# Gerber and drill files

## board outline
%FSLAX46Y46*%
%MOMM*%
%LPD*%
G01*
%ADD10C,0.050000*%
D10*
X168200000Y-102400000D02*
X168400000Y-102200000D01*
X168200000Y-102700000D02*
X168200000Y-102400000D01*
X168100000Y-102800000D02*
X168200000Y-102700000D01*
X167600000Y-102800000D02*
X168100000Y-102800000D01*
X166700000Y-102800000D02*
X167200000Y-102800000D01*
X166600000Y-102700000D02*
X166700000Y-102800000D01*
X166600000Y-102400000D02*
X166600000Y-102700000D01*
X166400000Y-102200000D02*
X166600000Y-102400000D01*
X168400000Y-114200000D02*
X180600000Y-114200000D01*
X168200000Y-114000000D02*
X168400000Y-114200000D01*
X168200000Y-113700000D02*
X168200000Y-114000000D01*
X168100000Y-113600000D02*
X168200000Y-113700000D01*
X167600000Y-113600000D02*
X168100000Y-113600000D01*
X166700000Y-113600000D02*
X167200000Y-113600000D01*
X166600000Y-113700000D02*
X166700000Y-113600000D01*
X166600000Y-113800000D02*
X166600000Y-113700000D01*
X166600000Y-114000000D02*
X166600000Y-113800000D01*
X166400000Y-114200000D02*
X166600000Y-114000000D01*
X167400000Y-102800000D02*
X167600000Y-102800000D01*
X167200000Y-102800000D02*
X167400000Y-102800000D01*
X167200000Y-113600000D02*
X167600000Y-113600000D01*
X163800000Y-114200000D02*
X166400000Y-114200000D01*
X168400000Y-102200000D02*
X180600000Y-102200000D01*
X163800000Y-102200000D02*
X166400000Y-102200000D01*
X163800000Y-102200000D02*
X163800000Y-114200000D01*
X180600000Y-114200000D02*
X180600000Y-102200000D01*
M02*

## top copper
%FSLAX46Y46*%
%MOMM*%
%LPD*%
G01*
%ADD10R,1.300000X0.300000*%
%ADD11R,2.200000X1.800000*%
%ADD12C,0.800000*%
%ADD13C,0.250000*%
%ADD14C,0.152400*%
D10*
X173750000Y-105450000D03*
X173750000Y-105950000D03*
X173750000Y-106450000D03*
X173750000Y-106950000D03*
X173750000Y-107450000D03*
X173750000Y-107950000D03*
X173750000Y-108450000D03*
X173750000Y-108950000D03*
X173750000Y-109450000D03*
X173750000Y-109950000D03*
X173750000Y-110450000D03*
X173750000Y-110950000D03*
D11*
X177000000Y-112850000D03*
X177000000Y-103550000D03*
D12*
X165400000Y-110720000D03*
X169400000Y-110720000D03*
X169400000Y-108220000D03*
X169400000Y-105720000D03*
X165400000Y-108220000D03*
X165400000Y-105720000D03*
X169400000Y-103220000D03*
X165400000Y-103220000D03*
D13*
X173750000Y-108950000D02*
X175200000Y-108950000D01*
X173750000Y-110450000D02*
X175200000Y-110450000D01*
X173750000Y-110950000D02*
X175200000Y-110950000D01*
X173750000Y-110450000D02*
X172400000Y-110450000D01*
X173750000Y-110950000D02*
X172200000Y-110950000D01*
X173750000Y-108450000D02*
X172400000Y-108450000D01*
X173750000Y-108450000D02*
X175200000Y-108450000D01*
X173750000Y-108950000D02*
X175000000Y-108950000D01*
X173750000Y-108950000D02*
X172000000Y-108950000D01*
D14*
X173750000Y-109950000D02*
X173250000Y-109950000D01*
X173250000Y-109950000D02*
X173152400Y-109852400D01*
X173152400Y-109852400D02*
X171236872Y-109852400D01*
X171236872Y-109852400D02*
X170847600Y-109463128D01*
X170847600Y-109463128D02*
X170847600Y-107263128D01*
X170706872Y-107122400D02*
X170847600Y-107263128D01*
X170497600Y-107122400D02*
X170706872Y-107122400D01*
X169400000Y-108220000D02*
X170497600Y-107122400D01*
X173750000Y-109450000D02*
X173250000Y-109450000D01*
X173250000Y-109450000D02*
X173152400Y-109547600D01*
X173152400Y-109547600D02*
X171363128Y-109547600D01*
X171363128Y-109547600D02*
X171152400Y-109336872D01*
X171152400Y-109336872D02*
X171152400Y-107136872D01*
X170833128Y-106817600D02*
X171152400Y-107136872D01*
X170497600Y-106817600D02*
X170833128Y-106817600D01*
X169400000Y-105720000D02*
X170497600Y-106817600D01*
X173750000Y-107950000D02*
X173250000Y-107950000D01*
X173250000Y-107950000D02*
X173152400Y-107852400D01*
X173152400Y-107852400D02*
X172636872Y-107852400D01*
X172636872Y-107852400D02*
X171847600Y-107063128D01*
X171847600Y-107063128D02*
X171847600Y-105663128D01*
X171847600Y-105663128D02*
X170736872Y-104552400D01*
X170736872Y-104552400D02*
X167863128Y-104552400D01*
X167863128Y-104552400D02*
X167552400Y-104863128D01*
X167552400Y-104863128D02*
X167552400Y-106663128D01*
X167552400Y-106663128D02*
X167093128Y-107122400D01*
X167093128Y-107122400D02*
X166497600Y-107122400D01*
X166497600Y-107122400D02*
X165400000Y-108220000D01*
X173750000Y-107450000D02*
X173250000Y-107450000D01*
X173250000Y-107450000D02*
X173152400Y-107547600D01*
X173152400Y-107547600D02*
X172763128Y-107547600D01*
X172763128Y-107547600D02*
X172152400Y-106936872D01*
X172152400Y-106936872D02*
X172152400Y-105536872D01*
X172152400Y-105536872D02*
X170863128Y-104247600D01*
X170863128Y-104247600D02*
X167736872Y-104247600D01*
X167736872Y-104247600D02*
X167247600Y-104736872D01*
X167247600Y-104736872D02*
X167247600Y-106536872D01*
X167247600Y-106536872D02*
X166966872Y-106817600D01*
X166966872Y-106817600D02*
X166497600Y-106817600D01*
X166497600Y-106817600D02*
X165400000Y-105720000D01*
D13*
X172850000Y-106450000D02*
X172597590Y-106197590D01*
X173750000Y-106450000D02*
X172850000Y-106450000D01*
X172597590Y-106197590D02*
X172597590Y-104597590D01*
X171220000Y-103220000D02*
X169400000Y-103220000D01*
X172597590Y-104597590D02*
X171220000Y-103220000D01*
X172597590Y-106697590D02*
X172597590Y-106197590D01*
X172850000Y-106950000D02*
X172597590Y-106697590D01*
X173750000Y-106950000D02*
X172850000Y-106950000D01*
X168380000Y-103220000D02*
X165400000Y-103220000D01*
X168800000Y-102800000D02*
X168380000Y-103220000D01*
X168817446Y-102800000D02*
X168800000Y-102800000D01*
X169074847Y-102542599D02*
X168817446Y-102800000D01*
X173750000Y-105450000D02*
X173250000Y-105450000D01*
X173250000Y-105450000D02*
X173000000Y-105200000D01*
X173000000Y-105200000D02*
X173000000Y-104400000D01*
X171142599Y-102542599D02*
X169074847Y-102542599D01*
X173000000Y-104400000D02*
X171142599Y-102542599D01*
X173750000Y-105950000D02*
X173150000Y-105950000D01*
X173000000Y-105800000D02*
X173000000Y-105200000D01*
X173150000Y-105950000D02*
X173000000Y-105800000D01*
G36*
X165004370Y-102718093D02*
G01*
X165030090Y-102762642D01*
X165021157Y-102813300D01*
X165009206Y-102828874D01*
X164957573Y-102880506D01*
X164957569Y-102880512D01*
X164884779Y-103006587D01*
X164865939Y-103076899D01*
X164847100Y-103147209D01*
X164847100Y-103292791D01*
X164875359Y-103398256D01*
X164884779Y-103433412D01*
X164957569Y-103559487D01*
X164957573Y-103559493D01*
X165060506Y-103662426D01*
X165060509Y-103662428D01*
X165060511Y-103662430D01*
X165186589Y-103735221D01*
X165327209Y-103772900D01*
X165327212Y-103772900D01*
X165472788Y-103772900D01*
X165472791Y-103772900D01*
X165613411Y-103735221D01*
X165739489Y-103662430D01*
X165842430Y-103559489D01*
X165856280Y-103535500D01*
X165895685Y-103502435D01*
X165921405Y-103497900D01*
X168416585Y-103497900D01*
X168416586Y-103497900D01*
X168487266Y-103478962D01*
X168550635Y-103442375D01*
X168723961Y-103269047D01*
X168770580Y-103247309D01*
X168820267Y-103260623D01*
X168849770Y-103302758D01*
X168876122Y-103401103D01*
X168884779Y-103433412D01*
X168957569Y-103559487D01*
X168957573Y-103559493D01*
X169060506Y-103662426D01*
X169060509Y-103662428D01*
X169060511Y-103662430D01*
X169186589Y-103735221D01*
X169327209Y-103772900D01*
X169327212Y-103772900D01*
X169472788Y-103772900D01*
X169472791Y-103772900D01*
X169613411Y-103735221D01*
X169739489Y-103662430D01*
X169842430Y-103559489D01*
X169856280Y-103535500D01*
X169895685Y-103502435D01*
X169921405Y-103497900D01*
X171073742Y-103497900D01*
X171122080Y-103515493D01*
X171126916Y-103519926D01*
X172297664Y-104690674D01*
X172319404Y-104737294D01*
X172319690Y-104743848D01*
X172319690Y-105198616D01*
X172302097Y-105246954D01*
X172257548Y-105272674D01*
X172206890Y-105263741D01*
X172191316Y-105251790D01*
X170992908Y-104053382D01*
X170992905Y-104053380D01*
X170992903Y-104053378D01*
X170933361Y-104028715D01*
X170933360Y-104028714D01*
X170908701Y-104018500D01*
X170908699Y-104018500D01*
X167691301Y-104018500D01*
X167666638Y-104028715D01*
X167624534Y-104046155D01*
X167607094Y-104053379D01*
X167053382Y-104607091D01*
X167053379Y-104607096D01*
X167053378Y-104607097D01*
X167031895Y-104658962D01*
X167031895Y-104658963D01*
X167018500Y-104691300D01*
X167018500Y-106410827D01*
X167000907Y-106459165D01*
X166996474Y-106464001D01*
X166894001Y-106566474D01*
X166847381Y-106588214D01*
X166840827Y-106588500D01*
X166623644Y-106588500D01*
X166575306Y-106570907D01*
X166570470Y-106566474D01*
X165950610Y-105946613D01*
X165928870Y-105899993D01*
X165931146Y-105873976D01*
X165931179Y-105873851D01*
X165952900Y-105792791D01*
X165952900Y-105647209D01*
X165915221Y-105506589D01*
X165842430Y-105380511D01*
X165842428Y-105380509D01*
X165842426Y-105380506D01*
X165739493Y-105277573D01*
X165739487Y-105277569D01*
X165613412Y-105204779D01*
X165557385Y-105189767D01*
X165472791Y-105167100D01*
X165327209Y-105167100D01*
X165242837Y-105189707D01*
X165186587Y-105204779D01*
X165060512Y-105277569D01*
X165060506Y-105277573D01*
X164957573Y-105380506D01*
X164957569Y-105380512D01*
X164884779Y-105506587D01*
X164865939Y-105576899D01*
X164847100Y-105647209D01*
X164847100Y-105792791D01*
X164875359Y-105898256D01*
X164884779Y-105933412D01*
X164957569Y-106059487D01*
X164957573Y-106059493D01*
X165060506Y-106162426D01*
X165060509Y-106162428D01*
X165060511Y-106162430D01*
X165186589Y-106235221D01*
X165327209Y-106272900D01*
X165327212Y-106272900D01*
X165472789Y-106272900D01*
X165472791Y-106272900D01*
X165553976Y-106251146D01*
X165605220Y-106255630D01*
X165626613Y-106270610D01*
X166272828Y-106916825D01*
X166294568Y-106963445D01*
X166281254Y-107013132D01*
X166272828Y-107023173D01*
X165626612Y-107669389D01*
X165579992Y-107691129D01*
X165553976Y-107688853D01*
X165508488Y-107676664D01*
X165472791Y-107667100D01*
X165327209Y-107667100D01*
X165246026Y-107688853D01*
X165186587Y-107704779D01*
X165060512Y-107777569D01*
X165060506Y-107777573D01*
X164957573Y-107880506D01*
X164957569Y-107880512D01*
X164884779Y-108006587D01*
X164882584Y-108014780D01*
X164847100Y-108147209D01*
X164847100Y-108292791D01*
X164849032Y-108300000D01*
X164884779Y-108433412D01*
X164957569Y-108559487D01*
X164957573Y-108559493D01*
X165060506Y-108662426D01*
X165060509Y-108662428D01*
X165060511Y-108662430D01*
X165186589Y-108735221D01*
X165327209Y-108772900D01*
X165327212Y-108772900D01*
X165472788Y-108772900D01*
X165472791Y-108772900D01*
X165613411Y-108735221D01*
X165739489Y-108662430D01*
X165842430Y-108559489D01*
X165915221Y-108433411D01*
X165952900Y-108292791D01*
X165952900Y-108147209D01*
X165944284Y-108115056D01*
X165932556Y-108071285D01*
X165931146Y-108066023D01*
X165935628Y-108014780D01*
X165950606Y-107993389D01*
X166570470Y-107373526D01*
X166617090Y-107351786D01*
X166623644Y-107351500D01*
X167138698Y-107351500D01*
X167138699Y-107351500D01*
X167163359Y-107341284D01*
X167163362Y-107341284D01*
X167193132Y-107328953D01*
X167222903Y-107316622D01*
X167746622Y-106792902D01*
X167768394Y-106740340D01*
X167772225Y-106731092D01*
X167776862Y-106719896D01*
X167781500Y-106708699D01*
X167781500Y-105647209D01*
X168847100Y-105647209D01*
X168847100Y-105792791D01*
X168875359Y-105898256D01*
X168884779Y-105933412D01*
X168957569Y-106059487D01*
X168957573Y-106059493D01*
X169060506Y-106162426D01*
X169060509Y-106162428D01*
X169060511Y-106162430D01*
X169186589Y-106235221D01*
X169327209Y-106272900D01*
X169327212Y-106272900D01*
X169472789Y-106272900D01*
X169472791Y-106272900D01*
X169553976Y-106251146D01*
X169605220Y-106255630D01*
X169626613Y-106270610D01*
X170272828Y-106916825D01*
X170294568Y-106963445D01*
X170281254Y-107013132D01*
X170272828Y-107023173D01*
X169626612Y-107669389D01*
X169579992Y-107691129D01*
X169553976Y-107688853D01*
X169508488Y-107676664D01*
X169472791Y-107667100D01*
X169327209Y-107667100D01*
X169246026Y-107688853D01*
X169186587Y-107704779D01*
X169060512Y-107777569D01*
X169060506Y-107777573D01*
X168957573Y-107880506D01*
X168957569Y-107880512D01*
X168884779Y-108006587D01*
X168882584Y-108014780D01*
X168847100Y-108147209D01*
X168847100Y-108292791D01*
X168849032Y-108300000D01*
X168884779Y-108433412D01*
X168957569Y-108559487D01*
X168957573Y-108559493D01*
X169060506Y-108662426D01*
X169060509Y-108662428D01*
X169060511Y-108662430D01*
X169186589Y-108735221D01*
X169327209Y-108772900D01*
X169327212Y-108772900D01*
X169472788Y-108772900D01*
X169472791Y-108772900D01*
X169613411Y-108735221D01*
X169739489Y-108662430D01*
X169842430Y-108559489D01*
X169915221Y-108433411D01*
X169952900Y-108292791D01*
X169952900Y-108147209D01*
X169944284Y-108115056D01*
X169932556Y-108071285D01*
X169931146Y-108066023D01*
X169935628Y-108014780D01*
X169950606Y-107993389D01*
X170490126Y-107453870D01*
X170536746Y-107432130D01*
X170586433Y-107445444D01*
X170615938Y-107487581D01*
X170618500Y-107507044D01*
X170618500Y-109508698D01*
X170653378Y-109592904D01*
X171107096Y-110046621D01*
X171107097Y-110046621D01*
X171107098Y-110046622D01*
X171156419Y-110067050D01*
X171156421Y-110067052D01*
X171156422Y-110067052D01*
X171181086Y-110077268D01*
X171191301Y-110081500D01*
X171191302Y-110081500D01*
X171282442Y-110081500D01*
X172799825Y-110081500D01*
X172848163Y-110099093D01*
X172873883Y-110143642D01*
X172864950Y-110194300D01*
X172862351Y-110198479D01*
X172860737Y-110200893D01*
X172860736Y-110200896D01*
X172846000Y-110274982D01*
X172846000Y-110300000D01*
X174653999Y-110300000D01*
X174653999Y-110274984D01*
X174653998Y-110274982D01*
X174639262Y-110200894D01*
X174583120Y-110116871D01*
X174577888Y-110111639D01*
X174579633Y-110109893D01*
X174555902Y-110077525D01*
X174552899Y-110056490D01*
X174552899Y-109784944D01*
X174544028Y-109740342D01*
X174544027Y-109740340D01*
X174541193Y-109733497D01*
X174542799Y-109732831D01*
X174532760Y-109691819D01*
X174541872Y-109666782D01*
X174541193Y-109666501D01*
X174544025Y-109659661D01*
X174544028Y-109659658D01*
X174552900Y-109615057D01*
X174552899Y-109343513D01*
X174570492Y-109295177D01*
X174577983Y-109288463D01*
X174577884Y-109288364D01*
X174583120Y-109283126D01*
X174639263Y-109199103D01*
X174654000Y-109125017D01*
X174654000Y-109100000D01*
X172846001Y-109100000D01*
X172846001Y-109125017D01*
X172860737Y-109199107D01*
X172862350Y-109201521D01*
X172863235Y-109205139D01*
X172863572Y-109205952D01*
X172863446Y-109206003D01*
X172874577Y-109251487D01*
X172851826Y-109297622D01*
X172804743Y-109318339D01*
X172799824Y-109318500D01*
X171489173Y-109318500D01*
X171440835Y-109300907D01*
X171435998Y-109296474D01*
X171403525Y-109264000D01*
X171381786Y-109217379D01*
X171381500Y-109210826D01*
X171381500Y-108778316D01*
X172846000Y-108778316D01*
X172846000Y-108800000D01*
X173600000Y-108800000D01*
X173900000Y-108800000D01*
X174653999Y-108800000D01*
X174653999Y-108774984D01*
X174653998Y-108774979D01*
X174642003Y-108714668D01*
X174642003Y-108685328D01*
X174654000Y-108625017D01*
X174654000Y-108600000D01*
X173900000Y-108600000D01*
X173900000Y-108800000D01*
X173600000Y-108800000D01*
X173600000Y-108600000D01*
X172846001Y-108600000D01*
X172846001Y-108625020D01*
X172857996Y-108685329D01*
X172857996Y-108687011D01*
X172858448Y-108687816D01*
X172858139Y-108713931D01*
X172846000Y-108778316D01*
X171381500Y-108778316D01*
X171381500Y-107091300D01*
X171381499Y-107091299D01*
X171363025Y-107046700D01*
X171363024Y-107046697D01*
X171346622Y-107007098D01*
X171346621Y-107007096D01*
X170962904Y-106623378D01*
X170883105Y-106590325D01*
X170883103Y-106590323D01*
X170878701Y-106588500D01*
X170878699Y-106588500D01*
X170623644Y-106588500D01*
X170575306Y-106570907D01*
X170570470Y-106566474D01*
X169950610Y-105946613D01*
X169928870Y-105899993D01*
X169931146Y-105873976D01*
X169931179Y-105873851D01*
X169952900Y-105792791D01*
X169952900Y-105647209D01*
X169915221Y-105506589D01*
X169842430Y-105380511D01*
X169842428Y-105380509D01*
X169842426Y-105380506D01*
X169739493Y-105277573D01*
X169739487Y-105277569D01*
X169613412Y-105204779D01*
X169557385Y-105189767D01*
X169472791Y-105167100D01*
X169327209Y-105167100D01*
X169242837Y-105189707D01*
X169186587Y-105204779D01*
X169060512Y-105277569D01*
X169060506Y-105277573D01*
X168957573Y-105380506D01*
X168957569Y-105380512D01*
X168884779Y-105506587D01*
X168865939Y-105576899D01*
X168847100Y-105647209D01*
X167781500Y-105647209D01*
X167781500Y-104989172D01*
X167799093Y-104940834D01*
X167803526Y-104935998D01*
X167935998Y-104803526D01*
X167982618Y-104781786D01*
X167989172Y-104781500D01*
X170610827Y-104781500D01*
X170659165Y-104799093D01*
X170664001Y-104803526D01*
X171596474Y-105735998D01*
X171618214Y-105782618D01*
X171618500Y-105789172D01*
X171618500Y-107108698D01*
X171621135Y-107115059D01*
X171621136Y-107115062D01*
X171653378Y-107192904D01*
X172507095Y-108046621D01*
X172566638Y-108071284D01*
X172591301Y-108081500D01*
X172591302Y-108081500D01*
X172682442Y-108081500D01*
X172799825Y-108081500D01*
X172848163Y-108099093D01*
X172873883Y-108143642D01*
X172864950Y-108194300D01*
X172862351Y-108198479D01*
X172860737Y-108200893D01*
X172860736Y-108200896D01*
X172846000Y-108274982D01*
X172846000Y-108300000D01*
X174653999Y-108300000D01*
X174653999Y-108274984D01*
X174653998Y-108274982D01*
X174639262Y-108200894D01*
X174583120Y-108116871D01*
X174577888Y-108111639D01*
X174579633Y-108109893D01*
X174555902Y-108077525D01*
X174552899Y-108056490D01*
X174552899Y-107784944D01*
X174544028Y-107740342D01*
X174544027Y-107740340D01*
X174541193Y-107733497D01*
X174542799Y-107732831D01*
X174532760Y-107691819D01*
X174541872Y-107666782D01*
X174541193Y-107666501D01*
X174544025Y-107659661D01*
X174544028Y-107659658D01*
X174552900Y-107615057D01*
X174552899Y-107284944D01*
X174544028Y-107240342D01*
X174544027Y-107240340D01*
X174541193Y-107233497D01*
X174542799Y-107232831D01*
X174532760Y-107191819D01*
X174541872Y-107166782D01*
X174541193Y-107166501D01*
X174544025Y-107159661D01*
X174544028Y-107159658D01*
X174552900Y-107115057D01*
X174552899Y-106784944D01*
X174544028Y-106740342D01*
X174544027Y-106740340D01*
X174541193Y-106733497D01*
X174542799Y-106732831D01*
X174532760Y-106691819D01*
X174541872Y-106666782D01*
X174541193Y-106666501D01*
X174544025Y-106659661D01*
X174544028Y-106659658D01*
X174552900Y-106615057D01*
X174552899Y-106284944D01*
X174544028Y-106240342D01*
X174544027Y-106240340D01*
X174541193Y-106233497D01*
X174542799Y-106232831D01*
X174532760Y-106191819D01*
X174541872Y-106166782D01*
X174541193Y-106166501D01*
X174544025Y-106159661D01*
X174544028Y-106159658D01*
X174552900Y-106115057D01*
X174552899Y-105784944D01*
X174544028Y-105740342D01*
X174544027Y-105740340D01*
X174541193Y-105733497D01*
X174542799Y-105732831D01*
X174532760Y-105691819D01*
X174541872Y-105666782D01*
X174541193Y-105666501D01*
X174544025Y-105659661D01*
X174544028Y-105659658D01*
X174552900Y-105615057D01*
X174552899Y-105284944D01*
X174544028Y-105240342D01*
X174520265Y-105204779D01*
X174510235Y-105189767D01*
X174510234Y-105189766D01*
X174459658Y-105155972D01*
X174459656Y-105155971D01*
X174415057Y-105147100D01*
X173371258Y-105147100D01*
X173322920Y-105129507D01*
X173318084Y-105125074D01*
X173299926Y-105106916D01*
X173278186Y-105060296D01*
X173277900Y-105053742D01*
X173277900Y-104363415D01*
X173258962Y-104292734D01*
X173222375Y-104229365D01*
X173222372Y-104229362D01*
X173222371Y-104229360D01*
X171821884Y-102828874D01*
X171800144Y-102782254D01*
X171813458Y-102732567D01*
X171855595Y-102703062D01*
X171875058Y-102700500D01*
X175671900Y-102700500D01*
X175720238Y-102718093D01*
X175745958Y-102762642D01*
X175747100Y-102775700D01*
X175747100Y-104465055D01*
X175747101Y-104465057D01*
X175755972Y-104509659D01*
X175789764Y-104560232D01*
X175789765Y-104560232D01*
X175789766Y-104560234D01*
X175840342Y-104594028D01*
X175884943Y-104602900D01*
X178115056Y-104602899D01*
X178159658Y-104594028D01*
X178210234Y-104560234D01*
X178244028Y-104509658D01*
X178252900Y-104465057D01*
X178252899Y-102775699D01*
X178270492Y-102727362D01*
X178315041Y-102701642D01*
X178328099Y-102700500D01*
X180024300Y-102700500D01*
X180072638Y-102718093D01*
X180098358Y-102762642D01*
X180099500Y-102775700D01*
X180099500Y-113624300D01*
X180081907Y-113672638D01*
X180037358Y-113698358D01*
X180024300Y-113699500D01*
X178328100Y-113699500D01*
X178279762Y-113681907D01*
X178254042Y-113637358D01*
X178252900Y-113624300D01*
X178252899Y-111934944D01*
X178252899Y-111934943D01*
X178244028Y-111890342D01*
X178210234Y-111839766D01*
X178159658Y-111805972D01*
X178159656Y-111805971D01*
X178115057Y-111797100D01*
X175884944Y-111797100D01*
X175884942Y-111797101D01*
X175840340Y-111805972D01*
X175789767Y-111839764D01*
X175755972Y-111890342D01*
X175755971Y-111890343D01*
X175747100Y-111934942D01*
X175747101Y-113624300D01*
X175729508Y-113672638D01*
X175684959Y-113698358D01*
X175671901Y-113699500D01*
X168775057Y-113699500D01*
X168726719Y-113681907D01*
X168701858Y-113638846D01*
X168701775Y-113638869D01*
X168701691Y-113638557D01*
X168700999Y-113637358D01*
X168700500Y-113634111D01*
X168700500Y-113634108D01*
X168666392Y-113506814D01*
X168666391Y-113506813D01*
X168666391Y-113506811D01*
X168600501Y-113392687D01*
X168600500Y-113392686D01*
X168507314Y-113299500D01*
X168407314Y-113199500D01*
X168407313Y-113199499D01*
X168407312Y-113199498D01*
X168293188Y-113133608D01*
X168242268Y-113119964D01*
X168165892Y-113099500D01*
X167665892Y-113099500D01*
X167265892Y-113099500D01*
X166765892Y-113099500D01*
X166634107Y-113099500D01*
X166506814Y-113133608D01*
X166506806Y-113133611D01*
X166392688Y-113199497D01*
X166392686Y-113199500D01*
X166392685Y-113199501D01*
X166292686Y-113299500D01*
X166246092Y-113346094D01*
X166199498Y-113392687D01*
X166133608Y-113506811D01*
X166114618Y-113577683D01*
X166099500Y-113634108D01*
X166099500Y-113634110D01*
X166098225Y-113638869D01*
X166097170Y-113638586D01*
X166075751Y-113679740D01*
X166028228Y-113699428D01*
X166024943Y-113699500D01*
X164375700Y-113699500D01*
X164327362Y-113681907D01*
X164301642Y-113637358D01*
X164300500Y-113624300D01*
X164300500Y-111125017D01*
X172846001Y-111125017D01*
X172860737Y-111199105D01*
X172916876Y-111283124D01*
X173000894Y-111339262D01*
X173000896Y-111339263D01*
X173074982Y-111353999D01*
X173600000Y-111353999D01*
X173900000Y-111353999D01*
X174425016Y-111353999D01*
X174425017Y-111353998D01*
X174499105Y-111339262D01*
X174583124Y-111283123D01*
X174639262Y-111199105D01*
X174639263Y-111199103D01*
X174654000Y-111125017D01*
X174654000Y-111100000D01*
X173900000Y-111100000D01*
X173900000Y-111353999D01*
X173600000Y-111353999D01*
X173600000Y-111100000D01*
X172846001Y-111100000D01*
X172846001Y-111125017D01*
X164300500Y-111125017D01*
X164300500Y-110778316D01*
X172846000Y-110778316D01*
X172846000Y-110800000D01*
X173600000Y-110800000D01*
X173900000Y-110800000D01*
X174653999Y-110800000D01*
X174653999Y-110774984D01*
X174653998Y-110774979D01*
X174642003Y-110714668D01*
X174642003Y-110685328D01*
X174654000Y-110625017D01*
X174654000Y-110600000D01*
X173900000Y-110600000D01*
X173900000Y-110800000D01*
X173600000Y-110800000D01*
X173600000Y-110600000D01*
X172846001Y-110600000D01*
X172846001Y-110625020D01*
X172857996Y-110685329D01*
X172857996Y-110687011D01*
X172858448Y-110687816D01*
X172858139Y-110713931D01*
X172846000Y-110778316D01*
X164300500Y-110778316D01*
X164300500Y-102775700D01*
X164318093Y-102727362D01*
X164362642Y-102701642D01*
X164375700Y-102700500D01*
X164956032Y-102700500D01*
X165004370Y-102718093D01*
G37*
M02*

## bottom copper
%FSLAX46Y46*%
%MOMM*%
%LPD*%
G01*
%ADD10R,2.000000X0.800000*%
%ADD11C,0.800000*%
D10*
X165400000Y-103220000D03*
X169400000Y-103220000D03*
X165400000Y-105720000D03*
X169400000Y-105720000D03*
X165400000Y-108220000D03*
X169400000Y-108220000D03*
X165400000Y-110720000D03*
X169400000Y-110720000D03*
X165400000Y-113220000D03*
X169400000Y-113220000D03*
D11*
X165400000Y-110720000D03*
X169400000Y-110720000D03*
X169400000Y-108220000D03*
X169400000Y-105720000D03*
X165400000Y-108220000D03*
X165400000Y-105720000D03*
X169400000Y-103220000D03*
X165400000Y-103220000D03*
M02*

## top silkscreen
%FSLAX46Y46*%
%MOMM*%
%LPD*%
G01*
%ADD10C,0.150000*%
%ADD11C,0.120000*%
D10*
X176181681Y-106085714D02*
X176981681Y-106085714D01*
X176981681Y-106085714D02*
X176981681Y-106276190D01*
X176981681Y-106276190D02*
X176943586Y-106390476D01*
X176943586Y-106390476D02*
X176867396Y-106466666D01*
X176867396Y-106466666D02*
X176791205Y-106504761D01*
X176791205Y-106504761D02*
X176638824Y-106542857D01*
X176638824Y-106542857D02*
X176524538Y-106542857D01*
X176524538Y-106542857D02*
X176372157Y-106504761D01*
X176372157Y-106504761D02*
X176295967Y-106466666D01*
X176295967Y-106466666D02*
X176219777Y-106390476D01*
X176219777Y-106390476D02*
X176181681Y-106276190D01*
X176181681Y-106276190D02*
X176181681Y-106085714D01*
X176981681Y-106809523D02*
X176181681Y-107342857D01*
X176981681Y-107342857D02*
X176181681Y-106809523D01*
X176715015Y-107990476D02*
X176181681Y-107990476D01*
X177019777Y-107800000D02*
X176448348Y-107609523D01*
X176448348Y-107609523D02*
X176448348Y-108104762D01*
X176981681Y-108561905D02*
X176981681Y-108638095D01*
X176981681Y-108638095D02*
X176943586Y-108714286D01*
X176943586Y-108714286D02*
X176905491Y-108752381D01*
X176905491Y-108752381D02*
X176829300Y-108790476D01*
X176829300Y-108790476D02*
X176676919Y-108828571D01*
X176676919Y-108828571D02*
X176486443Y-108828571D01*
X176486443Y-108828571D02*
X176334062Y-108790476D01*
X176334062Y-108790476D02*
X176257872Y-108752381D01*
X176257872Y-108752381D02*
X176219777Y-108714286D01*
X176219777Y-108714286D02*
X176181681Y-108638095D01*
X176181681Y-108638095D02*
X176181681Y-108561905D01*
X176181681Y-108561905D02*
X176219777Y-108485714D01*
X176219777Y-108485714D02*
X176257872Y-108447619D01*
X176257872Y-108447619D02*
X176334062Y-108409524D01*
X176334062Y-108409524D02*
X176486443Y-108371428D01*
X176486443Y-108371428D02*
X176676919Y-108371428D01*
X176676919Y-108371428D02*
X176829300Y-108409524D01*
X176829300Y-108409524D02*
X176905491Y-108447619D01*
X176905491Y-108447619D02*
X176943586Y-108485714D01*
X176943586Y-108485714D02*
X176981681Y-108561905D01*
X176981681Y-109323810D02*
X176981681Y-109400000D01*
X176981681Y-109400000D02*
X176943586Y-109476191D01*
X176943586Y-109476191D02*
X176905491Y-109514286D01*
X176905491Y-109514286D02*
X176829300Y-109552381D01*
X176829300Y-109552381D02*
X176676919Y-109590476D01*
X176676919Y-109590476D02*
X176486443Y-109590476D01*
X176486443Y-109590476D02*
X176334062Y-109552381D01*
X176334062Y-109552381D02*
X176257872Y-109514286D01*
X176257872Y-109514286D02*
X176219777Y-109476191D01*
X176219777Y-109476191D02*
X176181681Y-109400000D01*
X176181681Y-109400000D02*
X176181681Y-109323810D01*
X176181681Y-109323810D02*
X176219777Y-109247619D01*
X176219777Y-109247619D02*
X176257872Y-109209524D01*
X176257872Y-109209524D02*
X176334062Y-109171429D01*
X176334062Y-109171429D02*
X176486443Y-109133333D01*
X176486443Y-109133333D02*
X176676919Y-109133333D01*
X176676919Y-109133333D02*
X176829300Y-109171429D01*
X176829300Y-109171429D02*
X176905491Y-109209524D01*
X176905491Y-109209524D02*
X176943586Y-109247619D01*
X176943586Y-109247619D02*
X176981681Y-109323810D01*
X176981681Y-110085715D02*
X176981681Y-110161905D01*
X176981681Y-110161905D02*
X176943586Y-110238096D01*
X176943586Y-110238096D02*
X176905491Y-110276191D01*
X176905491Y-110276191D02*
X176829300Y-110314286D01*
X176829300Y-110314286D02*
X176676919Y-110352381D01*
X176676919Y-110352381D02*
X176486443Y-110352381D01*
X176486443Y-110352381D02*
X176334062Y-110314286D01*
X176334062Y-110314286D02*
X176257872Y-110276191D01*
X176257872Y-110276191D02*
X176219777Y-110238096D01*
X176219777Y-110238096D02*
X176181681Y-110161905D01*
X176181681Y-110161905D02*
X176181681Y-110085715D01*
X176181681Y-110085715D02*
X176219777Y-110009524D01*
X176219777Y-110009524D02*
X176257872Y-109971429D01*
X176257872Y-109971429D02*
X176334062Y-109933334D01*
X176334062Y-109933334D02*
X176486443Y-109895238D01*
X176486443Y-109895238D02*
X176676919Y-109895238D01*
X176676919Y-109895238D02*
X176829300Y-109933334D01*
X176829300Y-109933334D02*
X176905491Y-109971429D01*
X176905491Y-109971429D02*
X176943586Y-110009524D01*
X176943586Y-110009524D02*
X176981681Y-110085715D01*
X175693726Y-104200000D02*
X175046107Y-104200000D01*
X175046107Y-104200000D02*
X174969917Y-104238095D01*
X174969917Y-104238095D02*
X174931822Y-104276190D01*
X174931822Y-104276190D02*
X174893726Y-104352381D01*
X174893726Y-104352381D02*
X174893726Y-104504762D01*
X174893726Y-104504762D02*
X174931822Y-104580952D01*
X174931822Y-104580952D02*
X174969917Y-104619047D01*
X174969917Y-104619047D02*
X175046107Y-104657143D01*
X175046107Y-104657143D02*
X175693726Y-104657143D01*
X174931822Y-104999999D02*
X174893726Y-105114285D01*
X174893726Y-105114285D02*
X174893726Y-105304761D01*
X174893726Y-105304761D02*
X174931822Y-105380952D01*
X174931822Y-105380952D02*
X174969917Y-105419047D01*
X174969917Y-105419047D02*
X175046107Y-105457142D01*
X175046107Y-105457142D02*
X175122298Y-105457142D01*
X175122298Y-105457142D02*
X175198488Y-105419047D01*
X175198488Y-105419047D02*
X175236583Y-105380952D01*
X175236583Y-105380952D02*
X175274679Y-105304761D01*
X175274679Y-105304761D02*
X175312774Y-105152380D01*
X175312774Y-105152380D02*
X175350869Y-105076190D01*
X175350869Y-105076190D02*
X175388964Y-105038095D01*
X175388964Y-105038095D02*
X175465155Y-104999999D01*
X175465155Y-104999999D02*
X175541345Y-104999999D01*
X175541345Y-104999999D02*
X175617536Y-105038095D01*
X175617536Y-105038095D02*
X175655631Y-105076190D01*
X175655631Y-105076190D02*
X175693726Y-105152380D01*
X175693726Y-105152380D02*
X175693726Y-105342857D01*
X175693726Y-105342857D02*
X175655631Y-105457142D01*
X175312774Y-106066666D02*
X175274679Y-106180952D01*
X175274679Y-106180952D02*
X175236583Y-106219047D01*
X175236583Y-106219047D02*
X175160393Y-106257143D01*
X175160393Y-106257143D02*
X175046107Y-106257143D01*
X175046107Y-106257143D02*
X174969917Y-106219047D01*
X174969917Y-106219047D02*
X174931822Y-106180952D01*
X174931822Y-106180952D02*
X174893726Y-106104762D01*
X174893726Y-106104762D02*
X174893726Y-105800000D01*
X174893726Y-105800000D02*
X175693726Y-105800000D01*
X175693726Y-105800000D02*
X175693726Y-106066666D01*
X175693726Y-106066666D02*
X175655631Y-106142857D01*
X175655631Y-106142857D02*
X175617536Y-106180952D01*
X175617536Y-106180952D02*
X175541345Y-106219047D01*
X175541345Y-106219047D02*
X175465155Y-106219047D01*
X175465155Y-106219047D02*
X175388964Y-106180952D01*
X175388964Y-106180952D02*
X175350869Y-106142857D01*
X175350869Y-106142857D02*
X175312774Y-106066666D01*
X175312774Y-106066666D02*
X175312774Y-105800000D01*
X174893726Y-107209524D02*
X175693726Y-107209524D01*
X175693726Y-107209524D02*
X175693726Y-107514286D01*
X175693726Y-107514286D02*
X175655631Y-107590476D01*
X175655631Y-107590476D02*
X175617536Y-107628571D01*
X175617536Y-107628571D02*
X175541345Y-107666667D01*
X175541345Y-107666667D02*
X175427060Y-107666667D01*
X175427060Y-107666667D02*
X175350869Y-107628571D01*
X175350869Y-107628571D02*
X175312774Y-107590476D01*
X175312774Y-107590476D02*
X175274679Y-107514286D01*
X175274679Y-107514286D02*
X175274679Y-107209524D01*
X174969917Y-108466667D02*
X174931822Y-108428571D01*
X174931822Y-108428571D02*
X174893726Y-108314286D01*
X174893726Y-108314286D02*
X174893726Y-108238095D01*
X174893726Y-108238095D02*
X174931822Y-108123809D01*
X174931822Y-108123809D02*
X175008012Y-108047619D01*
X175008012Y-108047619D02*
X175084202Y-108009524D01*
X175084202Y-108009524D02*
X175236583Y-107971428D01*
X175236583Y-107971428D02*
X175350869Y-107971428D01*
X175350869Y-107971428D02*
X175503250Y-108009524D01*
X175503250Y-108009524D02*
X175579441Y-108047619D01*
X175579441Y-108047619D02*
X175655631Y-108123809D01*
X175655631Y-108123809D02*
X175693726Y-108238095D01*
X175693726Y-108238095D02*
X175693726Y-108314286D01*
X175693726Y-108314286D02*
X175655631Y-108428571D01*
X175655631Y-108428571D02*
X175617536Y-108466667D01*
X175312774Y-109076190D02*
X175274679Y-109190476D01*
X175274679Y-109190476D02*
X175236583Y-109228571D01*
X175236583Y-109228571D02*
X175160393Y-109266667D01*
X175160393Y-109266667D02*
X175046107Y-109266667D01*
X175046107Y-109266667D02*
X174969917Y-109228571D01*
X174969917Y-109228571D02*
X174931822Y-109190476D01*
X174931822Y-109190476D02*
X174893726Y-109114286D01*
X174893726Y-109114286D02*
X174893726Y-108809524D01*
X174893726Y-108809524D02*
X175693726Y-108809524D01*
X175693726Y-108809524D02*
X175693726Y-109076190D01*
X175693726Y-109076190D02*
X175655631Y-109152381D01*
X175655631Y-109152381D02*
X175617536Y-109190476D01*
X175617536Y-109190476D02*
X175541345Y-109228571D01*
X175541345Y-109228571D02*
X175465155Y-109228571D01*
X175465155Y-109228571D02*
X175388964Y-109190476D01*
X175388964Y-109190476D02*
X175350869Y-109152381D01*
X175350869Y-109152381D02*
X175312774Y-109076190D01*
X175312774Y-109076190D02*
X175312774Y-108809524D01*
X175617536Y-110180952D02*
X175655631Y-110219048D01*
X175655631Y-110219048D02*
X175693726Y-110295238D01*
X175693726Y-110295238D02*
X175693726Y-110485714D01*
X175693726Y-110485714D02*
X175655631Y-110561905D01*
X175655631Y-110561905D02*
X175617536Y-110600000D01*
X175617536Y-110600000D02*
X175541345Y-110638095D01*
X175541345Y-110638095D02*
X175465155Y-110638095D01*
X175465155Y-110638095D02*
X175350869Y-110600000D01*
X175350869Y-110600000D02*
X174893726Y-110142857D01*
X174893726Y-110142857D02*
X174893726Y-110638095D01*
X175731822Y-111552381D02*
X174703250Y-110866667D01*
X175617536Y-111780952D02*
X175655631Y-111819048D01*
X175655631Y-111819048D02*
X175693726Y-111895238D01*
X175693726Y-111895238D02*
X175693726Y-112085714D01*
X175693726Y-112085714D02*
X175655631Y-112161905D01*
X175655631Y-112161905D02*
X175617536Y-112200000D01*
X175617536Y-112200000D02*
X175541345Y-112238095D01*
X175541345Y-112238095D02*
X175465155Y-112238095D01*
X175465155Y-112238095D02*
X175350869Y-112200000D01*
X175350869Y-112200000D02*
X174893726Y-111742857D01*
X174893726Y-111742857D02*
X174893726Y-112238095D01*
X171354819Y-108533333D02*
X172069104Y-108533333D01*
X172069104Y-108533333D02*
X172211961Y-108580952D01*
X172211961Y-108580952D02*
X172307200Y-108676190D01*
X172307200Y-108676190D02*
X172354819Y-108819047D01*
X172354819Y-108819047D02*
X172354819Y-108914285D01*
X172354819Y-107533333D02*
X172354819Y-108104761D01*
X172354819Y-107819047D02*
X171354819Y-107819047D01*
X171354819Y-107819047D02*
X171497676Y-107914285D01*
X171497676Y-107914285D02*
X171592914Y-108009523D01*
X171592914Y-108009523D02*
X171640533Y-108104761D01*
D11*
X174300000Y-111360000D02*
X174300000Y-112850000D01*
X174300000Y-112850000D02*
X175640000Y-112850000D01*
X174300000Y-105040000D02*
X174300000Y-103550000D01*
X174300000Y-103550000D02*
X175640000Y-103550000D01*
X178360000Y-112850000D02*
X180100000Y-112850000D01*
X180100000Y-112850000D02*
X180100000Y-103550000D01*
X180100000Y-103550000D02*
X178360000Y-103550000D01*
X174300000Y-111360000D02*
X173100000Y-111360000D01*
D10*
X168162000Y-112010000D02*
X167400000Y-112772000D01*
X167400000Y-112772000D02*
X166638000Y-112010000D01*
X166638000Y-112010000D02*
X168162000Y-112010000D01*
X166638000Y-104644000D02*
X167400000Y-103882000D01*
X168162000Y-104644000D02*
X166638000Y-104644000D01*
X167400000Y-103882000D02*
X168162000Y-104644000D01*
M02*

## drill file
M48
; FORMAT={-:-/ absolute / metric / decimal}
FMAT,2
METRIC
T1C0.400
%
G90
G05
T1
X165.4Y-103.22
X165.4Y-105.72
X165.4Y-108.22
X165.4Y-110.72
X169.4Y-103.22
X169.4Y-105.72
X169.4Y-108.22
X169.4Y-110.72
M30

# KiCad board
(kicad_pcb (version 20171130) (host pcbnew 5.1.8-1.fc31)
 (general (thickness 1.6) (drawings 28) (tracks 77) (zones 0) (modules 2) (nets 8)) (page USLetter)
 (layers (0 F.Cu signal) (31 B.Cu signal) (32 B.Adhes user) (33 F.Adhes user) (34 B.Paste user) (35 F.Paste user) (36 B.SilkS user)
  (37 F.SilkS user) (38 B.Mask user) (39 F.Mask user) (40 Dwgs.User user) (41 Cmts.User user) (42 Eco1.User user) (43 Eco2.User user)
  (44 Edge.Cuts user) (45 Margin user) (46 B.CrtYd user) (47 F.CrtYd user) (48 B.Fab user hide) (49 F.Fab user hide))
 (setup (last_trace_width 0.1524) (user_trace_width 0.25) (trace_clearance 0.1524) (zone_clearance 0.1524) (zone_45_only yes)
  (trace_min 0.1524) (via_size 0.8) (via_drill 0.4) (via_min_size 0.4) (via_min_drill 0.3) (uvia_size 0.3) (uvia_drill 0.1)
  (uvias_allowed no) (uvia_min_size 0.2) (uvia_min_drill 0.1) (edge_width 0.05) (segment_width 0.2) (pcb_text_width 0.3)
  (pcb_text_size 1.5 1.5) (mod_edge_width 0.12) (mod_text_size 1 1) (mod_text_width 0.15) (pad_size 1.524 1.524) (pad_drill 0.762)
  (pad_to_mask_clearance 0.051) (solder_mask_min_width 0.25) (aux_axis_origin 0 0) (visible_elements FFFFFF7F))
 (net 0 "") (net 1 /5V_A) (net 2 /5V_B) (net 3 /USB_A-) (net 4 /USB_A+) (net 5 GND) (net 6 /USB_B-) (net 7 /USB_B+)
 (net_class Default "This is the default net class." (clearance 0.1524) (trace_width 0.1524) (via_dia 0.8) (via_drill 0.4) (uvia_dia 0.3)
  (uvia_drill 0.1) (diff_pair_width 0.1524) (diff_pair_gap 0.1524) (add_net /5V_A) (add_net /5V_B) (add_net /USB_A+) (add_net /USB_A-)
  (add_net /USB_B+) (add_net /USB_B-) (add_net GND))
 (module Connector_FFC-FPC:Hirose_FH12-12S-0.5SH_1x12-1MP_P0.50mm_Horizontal (layer F.Cu) (at 175.6 108.2 90)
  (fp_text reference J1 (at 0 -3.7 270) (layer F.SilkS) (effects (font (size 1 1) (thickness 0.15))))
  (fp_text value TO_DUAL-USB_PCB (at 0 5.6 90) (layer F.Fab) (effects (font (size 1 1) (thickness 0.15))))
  (fp_line (start -3.16 -1.3) (end -4.65 -1.3) (layer F.SilkS) (width 0.12))
  (fp_line (start -4.65 -1.3) (end -4.65 0.04) (layer F.SilkS) (width 0.12))
  (fp_line (start 3.16 -1.3) (end 4.65 -1.3) (layer F.SilkS) (width 0.12))
  (fp_line (start 4.65 -1.3) (end 4.65 0.04) (layer F.SilkS) (width 0.12))
  (fp_line (start -4.65 2.76) (end -4.65 4.5) (layer F.SilkS) (width 0.12))
  (fp_line (start -4.65 4.5) (end 4.65 4.5) (layer F.SilkS) (width 0.12))
  (fp_line (start 4.65 4.5) (end 4.65 2.76) (layer F.SilkS) (width 0.12))
  (fp_line (start -3.16 -1.3) (end -3.16 -2.5) (layer F.SilkS) (width 0.12))
  (pad 12 smd rect (at 2.75 -1.85 90) (size 0.3 1.3) (layers F.Cu F.Paste F.Mask) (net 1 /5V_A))
  (pad 11 smd rect (at 2.25 -1.85 90) (size 0.3 1.3) (layers F.Cu F.Paste F.Mask) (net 1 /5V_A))
  (pad 10 smd rect (at 1.75 -1.85 90) (size 0.3 1.3) (layers F.Cu F.Paste F.Mask) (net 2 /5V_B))
  (pad 9 smd rect (at 1.25 -1.85 90) (size 0.3 1.3) (layers F.Cu F.Paste F.Mask) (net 2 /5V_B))
  (pad 8 smd rect (at 0.75 -1.85 90) (size 0.3 1.3) (layers F.Cu F.Paste F.Mask) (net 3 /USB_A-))
  (pad 7 smd rect (at 0.25 -1.85 90) (size 0.3 1.3) (layers F.Cu F.Paste F.Mask) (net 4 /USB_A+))
  (pad 6 smd rect (at -0.25 -1.85 90) (size 0.3 1.3) (layers F.Cu F.Paste F.Mask) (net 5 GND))
  (pad 5 smd rect (at -0.75 -1.85 90) (size 0.3 1.3) (layers F.Cu F.Paste F.Mask) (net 5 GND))
  (pad 4 smd rect (at -1.25 -1.85 90) (size 0.3 1.3) (layers F.Cu F.Paste F.Mask) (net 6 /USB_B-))
  (pad 3 smd rect (at -1.75 -1.85 90) (size 0.3 1.3) (layers F.Cu F.Paste F.Mask) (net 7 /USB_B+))
  (pad 2 smd rect (at -2.25 -1.85 90) (size 0.3 1.3) (layers F.Cu F.Paste F.Mask) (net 5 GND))
  (pad 1 smd rect (at -2.75 -1.85 90) (size 0.3 1.3) (layers F.Cu F.Paste F.Mask) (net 5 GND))
  (pad MP smd rect (at -4.65 1.4 90) (size 1.8 2.2) (layers F.Cu F.Paste F.Mask))
  (pad MP smd rect (at 4.65 1.4 90) (size 1.8 2.2) (layers F.Cu F.Paste F.Mask)))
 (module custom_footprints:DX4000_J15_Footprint (layer B.Cu) (at 167.4 108.2 180)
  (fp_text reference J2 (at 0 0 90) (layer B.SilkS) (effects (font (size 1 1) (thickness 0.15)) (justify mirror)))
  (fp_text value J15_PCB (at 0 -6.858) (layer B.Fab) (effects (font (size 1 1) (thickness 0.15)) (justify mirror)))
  (fp_line (start -0.762 -3.81) (end 0 -4.572) (layer F.SilkS) (width 0.15))
  (fp_line (start 0 -4.572) (end 0.762 -3.81) (layer F.SilkS) (width 0.15))
  (fp_line (start 0.762 -3.81) (end -0.762 -3.81) (layer F.SilkS) (width 0.15))
  (fp_line (start 0.762 3.556) (end 0 4.318) (layer F.SilkS) (width 0.15))
  (fp_line (start -0.762 3.556) (end 0.762 3.556) (layer F.SilkS) (width 0.15))
  (fp_line (start 0 4.318) (end -0.762 3.556) (layer F.SilkS) (width 0.15))
  (pad 1 smd rect (at 2 4.98 180) (size 2 0.8) (layers B.Cu B.Paste B.Mask) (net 1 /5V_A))
  (pad 2 smd rect (at -2 4.98 180) (size 2 0.8) (layers B.Cu B.Paste B.Mask) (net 2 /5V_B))
  (pad 3 smd rect (at 2 2.48 180) (size 2 0.8) (layers B.Cu B.Paste B.Mask) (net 3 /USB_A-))
  (pad 4 smd rect (at -2 2.48 180) (size 2 0.8) (layers B.Cu B.Paste B.Mask) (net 6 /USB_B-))
  (pad 5 smd rect (at 2 -0.02 180) (size 2 0.8) (layers B.Cu B.Paste B.Mask) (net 4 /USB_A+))
  (pad 6 smd rect (at -2 -0.02 180) (size 2 0.8) (layers B.Cu B.Paste B.Mask) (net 7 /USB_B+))
  (pad 7 smd rect (at 2 -2.52 180) (size 2 0.8) (layers B.Cu B.Paste B.Mask) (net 5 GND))
  (pad 8 smd rect (at -2 -2.52 180) (size 2 0.8) (layers B.Cu B.Paste B.Mask) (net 5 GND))
  (pad 9 smd rect (at 2 -5.02 180) (size 2 0.8) (layers B.Cu B.Paste B.Mask))
  (pad 10 smd rect (at -2 -5.02 180) (size 2 0.8) (layers B.Cu B.Paste B.Mask)))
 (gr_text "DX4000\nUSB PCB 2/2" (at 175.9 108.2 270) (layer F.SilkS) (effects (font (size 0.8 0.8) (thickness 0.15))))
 (gr_line (start 168.2 102.4) (end 168.4 102.2) (layer Edge.Cuts) (width 0.05))
 (gr_line (start 168.2 102.7) (end 168.2 102.4) (layer Edge.Cuts) (width 0.05))
 (gr_line (start 168.1 102.8) (end 168.2 102.7) (layer Edge.Cuts) (width 0.05))
 (gr_line (start 167.6 102.8) (end 168.1 102.8) (layer Edge.Cuts) (width 0.05))
 (gr_line (start 166.7 102.8) (end 167.2 102.8) (layer Edge.Cuts) (width 0.05))
 (gr_line (start 166.6 102.7) (end 166.7 102.8) (layer Edge.Cuts) (width 0.05))
 (gr_line (start 166.6 102.4) (end 166.6 102.7) (layer Edge.Cuts) (width 0.05))
 (gr_line (start 166.4 102.2) (end 166.6 102.4) (layer Edge.Cuts) (width 0.05))
 (gr_line (start 168.4 114.2) (end 180.6 114.2) (layer Edge.Cuts) (width 0.05))
 (gr_line (start 168.2 114) (end 168.4 114.2) (layer Edge.Cuts) (width 0.05))
 (gr_line (start 168.2 113.7) (end 168.2 114) (layer Edge.Cuts) (width 0.05))
 (gr_line (start 168.1 113.6) (end 168.2 113.7) (layer Edge.Cuts) (width 0.05))
 (gr_line (start 167.6 113.6) (end 168.1 113.6) (layer Edge.Cuts) (width 0.05))
 (gr_line (start 166.7 113.6) (end 167.2 113.6) (layer Edge.Cuts) (width 0.05))
 (gr_line (start 166.6 113.7) (end 166.7 113.6) (layer Edge.Cuts) (width 0.05))
 (gr_line (start 166.6 113.8) (end 166.6 113.7) (layer Edge.Cuts) (width 0.05))
 (gr_line (start 166.6 114) (end 166.6 113.8) (layer Edge.Cuts) (width 0.05))
 (gr_line (start 166.4 114.2) (end 166.6 114) (layer Edge.Cuts) (width 0.05))
 (gr_line (start 167.4 102.8) (end 167.6 102.8) (layer Edge.Cuts) (width 0.05))
 (gr_line (start 167.2 102.8) (end 167.4 102.8) (layer Edge.Cuts) (width 0.05))
 (gr_line (start 167.2 113.6) (end 167.6 113.6) (layer Edge.Cuts) (width 0.05))
 (gr_line (start 163.8 114.2) (end 166.4 114.2) (layer Edge.Cuts) (width 0.05))
 (gr_line (start 168.4 102.2) (end 180.6 102.2) (layer Edge.Cuts) (width 0.05))
 (gr_line (start 163.8 102.2) (end 166.4 102.2) (layer Edge.Cuts) (width 0.05))
 (gr_line (start 163.8 102.2) (end 163.8 114.2) (layer Edge.Cuts) (width 0.05))
 (gr_line (start 180.6 114.2) (end 180.6 102.2) (layer Edge.Cuts) (width 0.05))
 (via (at 165.4 110.72) (size 0.8) (drill 0.4) (layers F.Cu B.Cu) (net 5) (status 40030))
 (via (at 169.4 110.72) (size 0.8) (drill 0.4) (layers F.Cu B.Cu) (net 5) (status 40030))
 (segment (start 173.75 108.95) (end 175.2 108.95) (width 0.25) (layer F.Cu) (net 5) (status 10))
 (segment (start 173.75 110.45) (end 175.2 110.45) (width 0.25) (layer F.Cu) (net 5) (status 10))
 (segment (start 173.75 110.95) (end 175.2 110.95) (width 0.25) (layer F.Cu) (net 5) (status 10))
 (segment (start 173.75 110.45) (end 172.4 110.45) (width 0.25) (layer F.Cu) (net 5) (status 10))
 (segment (start 173.75 110.95) (end 172.2 110.95) (width 0.25) (layer F.Cu) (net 5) (status 10))
 (segment (start 173.75 108.45) (end 172.4 108.45) (width 0.25) (layer F.Cu) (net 5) (status 10))
 (segment (start 173.75 108.45) (end 175.2 108.45) (width 0.25) (layer F.Cu) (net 5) (status 10))
 (segment (start 173.75 108.95) (end 175 108.95) (width 0.25) (layer F.Cu) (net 5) (status 10))
 (segment (start 173.75 108.95) (end 172 108.95) (width 0.25) (layer F.Cu) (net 5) (status 10))
 (segment (start 173.75 109.95) (end 173.25 109.95) (width 0.1524) (layer F.Cu) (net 7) (status 30))
 (segment (start 173.25 109.95) (end 173.1524 109.8524) (width 0.1524) (layer F.Cu) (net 7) (status 30))
 (segment (start 173.1524 109.8524) (end 171.236872 109.8524) (width 0.1524) (layer F.Cu) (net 7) (status 10))
 (segment (start 171.236872 109.8524) (end 170.8476 109.463128) (width 0.1524) (layer F.Cu) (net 7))
 (segment (start 170.8476 109.463128) (end 170.8476 107.263128) (width 0.1524) (layer F.Cu) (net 7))
 (segment (start 170.706872 107.1224) (end 170.8476 107.263128) (width 0.1524) (layer F.Cu) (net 7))
 (segment (start 170.4976 107.1224) (end 170.706872 107.1224) (width 0.1524) (layer F.Cu) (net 7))
 (segment (start 169.4 108.22) (end 170.4976 107.1224) (width 0.1524) (layer F.Cu) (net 7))
 (via (at 169.4 108.22) (size 0.8) (drill 0.4) (layers F.Cu B.Cu) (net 7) (status 40030))
 (segment (start 173.75 109.45) (end 173.25 109.45) (width 0.1524) (layer F.Cu) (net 6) (status 30))
 (segment (start 173.25 109.45) (end 173.1524 109.5476) (width 0.1524) (layer F.Cu) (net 6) (status 30))
 (segment (start 173.1524 109.5476) (end 171.363128 109.5476) (width 0.1524) (layer F.Cu) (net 6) (status 10))
 (segment (start 171.363128 109.5476) (end 171.1524 109.336872) (width 0.1524) (layer F.Cu) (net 6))
 (segment (start 171.1524 109.336872) (end 171.1524 107.136872) (width 0.1524) (layer F.Cu) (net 6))
 (segment (start 170.833128 106.8176) (end 171.1524 107.136872) (width 0.1524) (layer F.Cu) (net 6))
 (segment (start 170.4976 106.8176) (end 170.833128 106.8176) (width 0.1524) (layer F.Cu) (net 6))
 (segment (start 169.4 105.72) (end 170.4976 106.8176) (width 0.1524) (layer F.Cu) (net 6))
 (via (at 169.4 105.72) (size 0.8) (drill 0.4) (layers F.Cu B.Cu) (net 6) (status 40030))
 (segment (start 173.75 107.95) (end 173.25 107.95) (width 0.1524) (layer F.Cu) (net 4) (status 30))
 (segment (start 173.25 107.95) (end 173.1524 107.8524) (width 0.1524) (layer F.Cu) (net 4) (status 30))
 (segment (start 173.1524 107.8524) (end 172.636872 107.8524) (width 0.1524) (layer F.Cu) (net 4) (status 10))
 (segment (start 172.636872 107.8524) (end 171.8476 107.063128) (width 0.1524) (layer F.Cu) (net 4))
 (segment (start 171.8476 107.063128) (end 171.8476 105.663128) (width 0.1524) (layer F.Cu) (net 4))
 (segment (start 171.8476 105.663128) (end 170.736872 104.5524) (width 0.1524) (layer F.Cu) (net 4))
 (segment (start 170.736872 104.5524) (end 167.863128 104.5524) (width 0.1524) (layer F.Cu) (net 4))
 (segment (start 167.863128 104.5524) (end 167.5524 104.863128) (width 0.1524) (layer F.Cu) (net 4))
 (segment (start 167.5524 104.863128) (end 167.5524 106.663128) (width 0.1524) (layer F.Cu) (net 4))
 (segment (start 167.5524 106.663128) (end 167.093128 107.1224) (width 0.1524) (layer F.Cu) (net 4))
 (segment (start 167.093128 107.1224) (end 166.4976 107.1224) (width 0.1524) (layer F.Cu) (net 4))
 (segment (start 166.4976 107.1224) (end 165.4 108.22) (width 0.1524) (layer F.Cu) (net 4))
 (via (at 165.4 108.22) (size 0.8) (drill 0.4) (layers F.Cu B.Cu) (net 4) (status 40030))
 (segment (start 173.75 107.45) (end 173.25 107.45) (width 0.1524) (layer F.Cu) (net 3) (status 30))
 (segment (start 173.25 107.45) (end 173.1524 107.5476) (width 0.1524) (layer F.Cu) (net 3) (status 30))
 (segment (start 173.1524 107.5476) (end 172.763128 107.5476) (width 0.1524) (layer F.Cu) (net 3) (status 10))
 (segment (start 172.763128 107.5476) (end 172.1524 106.936872) (width 0.1524) (layer F.Cu) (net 3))
 (segment (start 172.1524 106.936872) (end 172.1524 105.536872) (width 0.1524) (layer F.Cu) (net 3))
 (segment (start 172.1524 105.536872) (end 170.863128 104.2476) (width 0.1524) (layer F.Cu) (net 3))
 (segment (start 170.863128 104.2476) (end 167.736872 104.2476) (width 0.1524) (layer F.Cu) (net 3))
 (segment (start 167.736872 104.2476) (end 167.2476 104.736872) (width 0.1524) (layer F.Cu) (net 3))
 (segment (start 167.2476 104.736872) (end 167.2476 106.536872) (width 0.1524) (layer F.Cu) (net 3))
 (segment (start 167.2476 106.536872) (end 166.966872 106.8176) (width 0.1524) (layer F.Cu) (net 3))
 (segment (start 166.966872 106.8176) (end 166.4976 106.8176) (width 0.1524) (layer F.Cu) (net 3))
 (segment (start 166.4976 106.8176) (end 165.4 105.72) (width 0.1524) (layer F.Cu) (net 3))
 (via (at 165.4 105.72) (size 0.8) (drill 0.4) (layers F.Cu B.Cu) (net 3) (status 40030))
 (via (at 169.4 103.22) (size 0.8) (drill 0.4) (layers F.Cu B.Cu) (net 2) (status 40030))
 (segment (start 172.85 106.45) (end 172.59759 106.19759) (width 0.25) (layer F.Cu) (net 2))
 (segment (start 173.75 106.45) (end 172.85 106.45) (width 0.25) (layer F.Cu) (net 2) (status 10))
 (segment (start 172.59759 106.19759) (end 172.59759 104.59759) (width 0.25) (layer F.Cu) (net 2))
 (segment (start 171.22 103.22) (end 169.4 103.22) (width 0.25) (layer F.Cu) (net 2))
 (segment (start 172.59759 104.59759) (end 171.22 103.22) (width 0.25) (layer F.Cu) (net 2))
 (segment (start 172.59759 106.69759) (end 172.59759 106.19759) (width 0.25) (layer F.Cu) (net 2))
 (segment (start 172.85 106.95) (end 172.59759 106.69759) (width 0.25) (layer F.Cu) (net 2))
 (segment (start 173.75 106.95) (end 172.85 106.95) (width 0.25) (layer F.Cu) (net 2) (status 10))
 (via (at 165.4 103.22) (size 0.8) (drill 0.4) (layers F.Cu B.Cu) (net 1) (status 40030))
 (segment (start 168.38 103.22) (end 165.4 103.22) (width 0.25) (layer F.Cu) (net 1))
 (segment (start 168.8 102.8) (end 168.38 103.22) (width 0.25) (layer F.Cu) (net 1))
 (segment (start 168.817446 102.8) (end 168.8 102.8) (width 0.25) (layer F.Cu) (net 1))
 (segment (start 169.074847 102.542599) (end 168.817446 102.8) (width 0.25) (layer F.Cu) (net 1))
 (segment (start 173.75 105.45) (end 173.25 105.45) (width 0.25) (layer F.Cu) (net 1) (status 30))
 (segment (start 173.25 105.45) (end 173 105.2) (width 0.25) (layer F.Cu) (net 1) (status 10))
 (segment (start 173 105.2) (end 173 104.4) (width 0.25) (layer F.Cu) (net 1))
 (segment (start 171.142599 102.542599) (end 169.074847 102.542599) (width 0.25) (layer F.Cu) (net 1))
 (segment (start 173 104.4) (end 171.142599 102.542599) (width 0.25) (layer F.Cu) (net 1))
 (segment (start 173.75 105.95) (end 173.15 105.95) (width 0.25) (layer F.Cu) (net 1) (status 30))
 (segment (start 173 105.8) (end 173 105.2) (width 0.25) (layer F.Cu) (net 1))
 (segment (start 173.15 105.95) (end 173 105.8) (width 0.25) (layer F.Cu) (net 1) (status 10))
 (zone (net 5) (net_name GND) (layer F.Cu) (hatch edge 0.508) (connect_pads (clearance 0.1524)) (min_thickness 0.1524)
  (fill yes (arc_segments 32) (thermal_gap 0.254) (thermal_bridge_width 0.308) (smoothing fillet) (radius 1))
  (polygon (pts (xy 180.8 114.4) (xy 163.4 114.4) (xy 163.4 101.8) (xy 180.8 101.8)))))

